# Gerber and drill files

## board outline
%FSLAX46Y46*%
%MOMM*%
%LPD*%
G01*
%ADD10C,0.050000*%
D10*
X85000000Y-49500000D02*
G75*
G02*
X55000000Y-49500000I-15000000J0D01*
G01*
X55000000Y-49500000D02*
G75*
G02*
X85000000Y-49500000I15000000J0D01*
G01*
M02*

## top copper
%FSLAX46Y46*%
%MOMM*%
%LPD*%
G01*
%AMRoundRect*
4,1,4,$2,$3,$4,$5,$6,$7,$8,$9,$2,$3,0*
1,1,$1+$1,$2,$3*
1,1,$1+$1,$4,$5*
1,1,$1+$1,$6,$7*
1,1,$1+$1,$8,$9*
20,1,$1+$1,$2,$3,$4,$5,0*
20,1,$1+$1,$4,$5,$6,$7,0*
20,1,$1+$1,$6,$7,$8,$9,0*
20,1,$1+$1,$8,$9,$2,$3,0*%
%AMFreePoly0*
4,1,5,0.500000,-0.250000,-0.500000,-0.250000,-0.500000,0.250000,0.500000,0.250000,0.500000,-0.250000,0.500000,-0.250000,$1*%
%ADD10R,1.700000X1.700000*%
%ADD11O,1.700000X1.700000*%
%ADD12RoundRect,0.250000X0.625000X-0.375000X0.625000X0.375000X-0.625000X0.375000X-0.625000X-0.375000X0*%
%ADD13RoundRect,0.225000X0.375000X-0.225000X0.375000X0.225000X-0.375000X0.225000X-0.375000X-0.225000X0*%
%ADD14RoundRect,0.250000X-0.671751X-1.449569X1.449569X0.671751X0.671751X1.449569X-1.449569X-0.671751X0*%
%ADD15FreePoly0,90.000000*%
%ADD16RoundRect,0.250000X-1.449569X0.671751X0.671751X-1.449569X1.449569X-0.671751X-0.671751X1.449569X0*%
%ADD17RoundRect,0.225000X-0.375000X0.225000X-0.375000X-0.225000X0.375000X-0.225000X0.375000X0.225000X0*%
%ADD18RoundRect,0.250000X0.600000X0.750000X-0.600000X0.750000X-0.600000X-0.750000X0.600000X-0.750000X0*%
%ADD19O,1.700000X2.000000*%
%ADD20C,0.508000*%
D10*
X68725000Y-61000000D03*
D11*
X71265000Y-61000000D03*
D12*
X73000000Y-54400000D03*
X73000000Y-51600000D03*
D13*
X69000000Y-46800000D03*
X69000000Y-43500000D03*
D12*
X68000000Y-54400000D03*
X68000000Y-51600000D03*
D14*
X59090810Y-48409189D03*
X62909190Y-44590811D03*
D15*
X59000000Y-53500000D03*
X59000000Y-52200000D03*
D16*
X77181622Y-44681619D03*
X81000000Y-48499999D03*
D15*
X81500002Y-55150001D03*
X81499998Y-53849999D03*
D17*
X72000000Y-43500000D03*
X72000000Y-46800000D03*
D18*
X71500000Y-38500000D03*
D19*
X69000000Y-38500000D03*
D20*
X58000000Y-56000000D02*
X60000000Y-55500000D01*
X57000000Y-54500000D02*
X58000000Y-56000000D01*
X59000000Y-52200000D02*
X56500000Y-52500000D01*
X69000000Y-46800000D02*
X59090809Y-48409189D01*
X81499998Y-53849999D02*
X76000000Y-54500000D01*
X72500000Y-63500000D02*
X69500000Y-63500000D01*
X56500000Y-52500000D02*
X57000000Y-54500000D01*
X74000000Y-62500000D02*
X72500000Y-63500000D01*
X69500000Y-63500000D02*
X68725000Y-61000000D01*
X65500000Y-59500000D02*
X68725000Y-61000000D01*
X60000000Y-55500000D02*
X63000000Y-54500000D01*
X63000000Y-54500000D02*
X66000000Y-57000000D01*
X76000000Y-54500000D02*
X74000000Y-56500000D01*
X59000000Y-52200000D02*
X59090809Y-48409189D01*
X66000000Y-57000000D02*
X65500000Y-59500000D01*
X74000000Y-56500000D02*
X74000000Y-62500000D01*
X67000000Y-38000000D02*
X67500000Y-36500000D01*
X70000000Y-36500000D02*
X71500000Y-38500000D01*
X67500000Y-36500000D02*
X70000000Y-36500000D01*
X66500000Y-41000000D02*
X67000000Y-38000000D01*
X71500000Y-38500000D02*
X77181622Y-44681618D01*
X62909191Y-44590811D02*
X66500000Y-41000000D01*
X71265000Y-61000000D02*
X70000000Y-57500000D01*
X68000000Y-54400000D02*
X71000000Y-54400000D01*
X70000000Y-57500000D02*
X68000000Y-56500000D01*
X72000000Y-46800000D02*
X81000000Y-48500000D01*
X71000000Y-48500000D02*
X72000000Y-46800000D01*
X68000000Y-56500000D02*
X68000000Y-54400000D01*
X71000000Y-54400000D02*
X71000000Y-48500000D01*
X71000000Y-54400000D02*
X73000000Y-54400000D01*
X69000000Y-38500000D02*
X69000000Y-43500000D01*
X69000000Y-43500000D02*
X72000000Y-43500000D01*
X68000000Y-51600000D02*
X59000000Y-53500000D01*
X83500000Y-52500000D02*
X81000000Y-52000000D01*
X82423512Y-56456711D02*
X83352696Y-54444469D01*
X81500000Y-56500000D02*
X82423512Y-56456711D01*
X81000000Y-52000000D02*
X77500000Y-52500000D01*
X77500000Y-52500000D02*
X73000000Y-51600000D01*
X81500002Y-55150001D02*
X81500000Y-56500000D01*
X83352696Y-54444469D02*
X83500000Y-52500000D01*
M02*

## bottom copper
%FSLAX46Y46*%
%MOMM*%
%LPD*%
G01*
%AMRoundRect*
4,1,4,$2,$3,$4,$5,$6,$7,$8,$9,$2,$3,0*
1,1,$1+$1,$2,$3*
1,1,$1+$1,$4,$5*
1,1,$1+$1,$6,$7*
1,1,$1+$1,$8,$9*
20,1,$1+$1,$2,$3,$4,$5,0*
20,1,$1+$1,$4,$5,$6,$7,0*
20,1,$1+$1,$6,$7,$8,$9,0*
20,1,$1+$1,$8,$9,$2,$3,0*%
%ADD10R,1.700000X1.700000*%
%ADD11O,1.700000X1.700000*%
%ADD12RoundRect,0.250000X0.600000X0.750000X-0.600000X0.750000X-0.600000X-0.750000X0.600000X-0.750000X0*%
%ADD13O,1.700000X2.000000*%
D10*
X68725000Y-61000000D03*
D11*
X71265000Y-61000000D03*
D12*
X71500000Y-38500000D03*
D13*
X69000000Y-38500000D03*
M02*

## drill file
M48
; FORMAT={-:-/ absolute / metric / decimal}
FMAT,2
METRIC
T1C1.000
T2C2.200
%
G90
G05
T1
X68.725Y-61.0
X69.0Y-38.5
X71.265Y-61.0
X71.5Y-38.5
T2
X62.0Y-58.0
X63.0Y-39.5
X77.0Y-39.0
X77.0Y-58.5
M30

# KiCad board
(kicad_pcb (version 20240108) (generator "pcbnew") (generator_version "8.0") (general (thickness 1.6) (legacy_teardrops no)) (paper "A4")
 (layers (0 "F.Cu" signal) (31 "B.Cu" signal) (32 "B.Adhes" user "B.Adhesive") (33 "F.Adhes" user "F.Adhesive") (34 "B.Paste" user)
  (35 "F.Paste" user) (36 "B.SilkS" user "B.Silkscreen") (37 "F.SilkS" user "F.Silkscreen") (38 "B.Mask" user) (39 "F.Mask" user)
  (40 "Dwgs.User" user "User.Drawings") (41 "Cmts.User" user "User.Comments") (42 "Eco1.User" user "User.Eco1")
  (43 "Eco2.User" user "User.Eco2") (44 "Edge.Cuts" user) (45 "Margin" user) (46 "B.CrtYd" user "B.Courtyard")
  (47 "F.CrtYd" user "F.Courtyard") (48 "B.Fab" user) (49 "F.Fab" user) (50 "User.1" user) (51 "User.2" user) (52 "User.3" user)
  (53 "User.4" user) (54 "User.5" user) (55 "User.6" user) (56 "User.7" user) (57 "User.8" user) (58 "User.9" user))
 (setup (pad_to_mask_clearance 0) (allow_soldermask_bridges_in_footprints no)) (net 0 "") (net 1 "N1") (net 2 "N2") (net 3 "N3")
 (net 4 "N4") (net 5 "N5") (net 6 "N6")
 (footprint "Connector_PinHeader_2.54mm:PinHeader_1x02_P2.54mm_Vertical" (layer "F.Cu") (at 68.725 61 90)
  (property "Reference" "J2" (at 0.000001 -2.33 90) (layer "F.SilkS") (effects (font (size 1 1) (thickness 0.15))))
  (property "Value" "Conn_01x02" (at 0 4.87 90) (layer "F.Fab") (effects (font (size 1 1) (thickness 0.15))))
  (pad "1" thru_hole rect (at 0 0 90) (size 1.7 1.7) (drill 1) (layers "*.Cu" "*.Mask") (remove_unused_layers no) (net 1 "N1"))
  (pad "2" thru_hole oval (at 0 2.54 90) (size 1.7 1.7) (drill 1) (layers "*.Cu" "*.Mask") (remove_unused_layers no) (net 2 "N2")))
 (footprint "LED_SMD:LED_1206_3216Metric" (layer "F.Cu") (at 73 53 90)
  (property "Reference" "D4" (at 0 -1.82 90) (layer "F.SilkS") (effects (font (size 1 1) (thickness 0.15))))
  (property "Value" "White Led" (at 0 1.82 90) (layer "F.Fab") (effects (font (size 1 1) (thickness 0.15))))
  (pad "1" smd roundrect (at -1.4 0 90) (size 1.25 1.75) (layers "F.Cu" "F.Paste" "F.Mask") (roundrect_rratio 0.2) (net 2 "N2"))
  (pad "2" smd roundrect (at 1.4 0 90) (size 1.25 1.75) (layers "F.Cu" "F.Paste" "F.Mask") (roundrect_rratio 0.2) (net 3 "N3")))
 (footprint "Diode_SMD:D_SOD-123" (layer "F.Cu") (at 69 45.15 90)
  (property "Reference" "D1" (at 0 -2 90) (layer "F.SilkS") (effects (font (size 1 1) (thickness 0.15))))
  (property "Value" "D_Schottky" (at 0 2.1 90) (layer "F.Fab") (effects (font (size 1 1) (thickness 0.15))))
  (pad "1" smd roundrect (at -1.65 0 90) (size 0.9 1.2) (layers "F.Cu" "F.Paste" "F.Mask") (roundrect_rratio 0.25) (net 1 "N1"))
  (pad "2" smd roundrect (at 1.65 0 90) (size 0.9 1.2) (layers "F.Cu" "F.Paste" "F.Mask") (roundrect_rratio 0.25) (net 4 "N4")))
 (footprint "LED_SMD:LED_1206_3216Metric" (layer "F.Cu") (at 68 53 90)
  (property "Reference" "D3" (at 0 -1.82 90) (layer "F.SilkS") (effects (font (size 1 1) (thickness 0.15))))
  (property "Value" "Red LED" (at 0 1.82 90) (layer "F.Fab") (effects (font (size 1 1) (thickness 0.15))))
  (pad "1" smd roundrect (at -1.4 0 90) (size 1.25 1.75) (layers "F.Cu" "F.Paste" "F.Mask") (roundrect_rratio 0.2) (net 2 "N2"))
  (pad "2" smd roundrect (at 1.4 0 90) (size 1.25 1.75) (layers "F.Cu" "F.Paste" "F.Mask") (roundrect_rratio 0.2) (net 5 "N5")))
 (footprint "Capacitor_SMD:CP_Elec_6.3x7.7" (layer "F.Cu") (at 61 46.5 45)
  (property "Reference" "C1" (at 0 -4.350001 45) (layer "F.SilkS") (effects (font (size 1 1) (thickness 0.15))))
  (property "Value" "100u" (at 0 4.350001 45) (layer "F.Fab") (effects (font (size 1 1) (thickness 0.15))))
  (pad "1" smd roundrect (at -2.700002 -0.000001 45) (size 3.5 1.6) (layers "F.Cu" "F.Paste" "F.Mask") (roundrect_rratio 0.15625)
   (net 1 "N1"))
  (pad "2" smd roundrect (at 2.700002 0.000001 45) (size 3.5 1.6) (layers "F.Cu" "F.Paste" "F.Mask") (roundrect_rratio 0.15625) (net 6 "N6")))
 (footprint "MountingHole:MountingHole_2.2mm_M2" (layer "F.Cu") (at 62 58)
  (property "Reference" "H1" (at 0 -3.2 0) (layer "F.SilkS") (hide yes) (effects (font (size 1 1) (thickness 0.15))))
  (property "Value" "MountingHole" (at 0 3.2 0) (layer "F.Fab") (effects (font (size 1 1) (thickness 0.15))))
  (pad "" np_thru_hole circle (at 0 0) (size 2.2 2.2) (drill 2.2) (layers "*.Cu" "*.Mask")))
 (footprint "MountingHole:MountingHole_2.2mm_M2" (layer "F.Cu") (at 77 39)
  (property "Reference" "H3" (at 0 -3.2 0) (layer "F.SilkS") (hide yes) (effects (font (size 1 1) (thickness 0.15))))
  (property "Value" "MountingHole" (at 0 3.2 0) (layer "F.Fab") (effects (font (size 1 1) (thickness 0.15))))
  (pad "" np_thru_hole circle (at 0 0) (size 2.2 2.2) (drill 2.2) (layers "*.Cu" "*.Mask")))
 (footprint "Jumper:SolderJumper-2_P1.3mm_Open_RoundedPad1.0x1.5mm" (layer "F.Cu") (at 59 52.85 90)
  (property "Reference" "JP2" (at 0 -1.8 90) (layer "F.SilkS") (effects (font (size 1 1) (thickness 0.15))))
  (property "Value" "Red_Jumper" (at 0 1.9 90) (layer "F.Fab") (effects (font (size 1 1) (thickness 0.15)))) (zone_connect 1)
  (pad "1" smd custom (at -0.65 0 90) (size 1 0.5) (layers "F.Cu" "F.Mask") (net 5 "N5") (zone_connect 2) (thermal_bridge_angle 45)
   (options (clearance outline) (anchor rect)) (primitives))
  (pad "2" smd custom (at 0.65 0 90) (size 1 0.5) (layers "F.Cu" "F.Mask") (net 1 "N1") (zone_connect 2) (thermal_bridge_angle 45)
   (options (clearance outline) (anchor rect)) (primitives)))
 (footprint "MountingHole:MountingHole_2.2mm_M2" (layer "F.Cu") (at 77 58.5)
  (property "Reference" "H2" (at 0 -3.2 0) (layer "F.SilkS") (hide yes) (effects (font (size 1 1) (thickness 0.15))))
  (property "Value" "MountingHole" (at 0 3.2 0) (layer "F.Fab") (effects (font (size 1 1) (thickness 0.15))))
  (pad "" np_thru_hole circle (at 0 0) (size 2.2 2.2) (drill 2.2) (layers "*.Cu" "*.Mask")))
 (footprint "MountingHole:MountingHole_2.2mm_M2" (layer "F.Cu") (at 63 39.5)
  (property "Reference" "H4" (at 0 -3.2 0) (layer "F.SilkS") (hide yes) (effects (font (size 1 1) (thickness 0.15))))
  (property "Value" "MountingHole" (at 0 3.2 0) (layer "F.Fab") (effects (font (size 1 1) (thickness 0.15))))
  (pad "" np_thru_hole circle (at 0 0) (size 2.2 2.2) (drill 2.2) (layers "*.Cu" "*.Mask")))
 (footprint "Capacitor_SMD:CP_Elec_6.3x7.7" (layer "F.Cu") (at 79.090811 46.590809 -45)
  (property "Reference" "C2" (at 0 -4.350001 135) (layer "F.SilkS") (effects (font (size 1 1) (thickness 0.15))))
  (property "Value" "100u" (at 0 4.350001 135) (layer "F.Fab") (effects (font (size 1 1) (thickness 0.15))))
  (pad "1" smd roundrect (at -2.700002 -0.000001 315) (size 3.5 1.6) (layers "F.Cu" "F.Paste" "F.Mask") (roundrect_rratio 0.15625)
   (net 6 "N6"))
  (pad "2" smd roundrect (at 2.700002 0.000001 315) (size 3.5 1.6) (layers "F.Cu" "F.Paste" "F.Mask") (roundrect_rratio 0.15625)
   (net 2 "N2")))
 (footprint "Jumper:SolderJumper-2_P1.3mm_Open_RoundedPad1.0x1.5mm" (layer "F.Cu") (at 81.5 54.5 90)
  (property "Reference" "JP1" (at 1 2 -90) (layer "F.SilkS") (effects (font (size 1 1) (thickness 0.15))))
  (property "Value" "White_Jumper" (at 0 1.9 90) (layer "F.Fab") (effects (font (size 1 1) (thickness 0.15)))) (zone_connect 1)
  (pad "1" smd custom (at -0.650001 0.000002 90) (size 1 0.5) (layers "F.Cu" "F.Mask") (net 3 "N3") (zone_connect 2)
   (thermal_bridge_angle 45) (options (clearance outline) (anchor rect)) (primitives))
  (pad "2" smd custom (at 0.650001 -0.000002 90) (size 1 0.5) (layers "F.Cu" "F.Mask") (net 1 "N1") (zone_connect 2)
   (thermal_bridge_angle 45) (options (clearance outline) (anchor rect)) (primitives)))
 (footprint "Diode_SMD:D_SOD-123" (layer "F.Cu") (at 72 45.15 -90)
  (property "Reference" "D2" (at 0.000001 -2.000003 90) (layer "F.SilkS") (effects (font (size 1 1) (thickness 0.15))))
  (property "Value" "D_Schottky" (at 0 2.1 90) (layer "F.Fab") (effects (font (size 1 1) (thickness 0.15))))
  (pad "1" smd roundrect (at -1.65 0 270) (size 0.9 1.2) (layers "F.Cu" "F.Paste" "F.Mask") (roundrect_rratio 0.25) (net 4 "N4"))
  (pad "2" smd roundrect (at 1.65 0 270) (size 0.9 1.2) (layers "F.Cu" "F.Paste" "F.Mask") (roundrect_rratio 0.25) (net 2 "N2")))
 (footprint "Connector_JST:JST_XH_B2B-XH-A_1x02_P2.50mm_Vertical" (layer "B.Cu") (at 71.5 38.5 180)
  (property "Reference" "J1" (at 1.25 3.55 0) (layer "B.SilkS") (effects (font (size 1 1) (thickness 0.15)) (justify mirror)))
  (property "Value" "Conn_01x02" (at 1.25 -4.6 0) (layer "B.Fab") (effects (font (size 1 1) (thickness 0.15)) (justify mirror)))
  (pad "1" thru_hole roundrect (at 0 0 180) (size 1.7 2) (drill 1) (layers "*.Cu" "*.Mask") (remove_unused_layers no)
   (roundrect_rratio 0.147059) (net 6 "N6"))
  (pad "2" thru_hole oval (at 2.5 0 180) (size 1.7 2) (drill 1) (layers "*.Cu" "*.Mask") (remove_unused_layers no) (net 4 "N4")))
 (gr_circle (center 70 49.5) (end 85 49.5) (stroke (width 0.05) (type default)) (fill none) (layer "Edge.Cuts"))
 (segment (start 58 56) (end 60 55.5) (width 0.508) (layer "F.Cu") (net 1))
 (segment (start 57 54.5) (end 58 56) (width 0.508) (layer "F.Cu") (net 1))
 (segment (start 59 52.2) (end 56.5 52.5) (width 0.508) (layer "F.Cu") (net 1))
 (segment (start 69 46.8) (end 59.090809 48.409189) (width 0.508) (layer "F.Cu") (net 1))
 (segment (start 81.499998 53.849999) (end 76 54.5) (width 0.508) (layer "F.Cu") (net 1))
 (segment (start 72.5 63.5) (end 69.5 63.5) (width 0.508) (layer "F.Cu") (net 1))
 (segment (start 56.5 52.5) (end 57 54.5) (width 0.508) (layer "F.Cu") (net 1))
 (segment (start 74 62.5) (end 72.5 63.5) (width 0.508) (layer "F.Cu") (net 1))
 (segment (start 69.5 63.5) (end 68.725 61) (width 0.508) (layer "F.Cu") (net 1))
 (segment (start 65.5 59.5) (end 68.725 61) (width 0.508) (layer "F.Cu") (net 1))
 (segment (start 60 55.5) (end 63 54.5) (width 0.508) (layer "F.Cu") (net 1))
 (segment (start 63 54.5) (end 66 57) (width 0.508) (layer "F.Cu") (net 1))
 (segment (start 76 54.5) (end 74 56.5) (width 0.508) (layer "F.Cu") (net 1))
 (segment (start 59 52.2) (end 59.090809 48.409189) (width 0.508) (layer "F.Cu") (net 1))
 (segment (start 66 57) (end 65.5 59.5) (width 0.508) (layer "F.Cu") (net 1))
 (segment (start 74 56.5) (end 74 62.5) (width 0.508) (layer "F.Cu") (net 1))
 (segment (start 67 38) (end 67.5 36.5) (width 0.508) (layer "F.Cu") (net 6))
 (segment (start 70 36.5) (end 71.5 38.5) (width 0.508) (layer "F.Cu") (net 6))
 (segment (start 67.5 36.5) (end 70 36.5) (width 0.508) (layer "F.Cu") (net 6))
 (segment (start 66.5 41) (end 67 38) (width 0.508) (layer "F.Cu") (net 6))
 (segment (start 71.5 38.5) (end 77.181622 44.681618) (width 0.508) (layer "F.Cu") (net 6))
 (segment (start 62.909191 44.590811) (end 66.5 41) (width 0.508) (layer "F.Cu") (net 6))
 (segment (start 71.265 61) (end 70 57.5) (width 0.508) (layer "F.Cu") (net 2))
 (segment (start 68 54.4) (end 71 54.4) (width 0.508) (layer "F.Cu") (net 2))
 (segment (start 70 57.5) (end 68 56.5) (width 0.508) (layer "F.Cu") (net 2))
 (segment (start 72 46.8) (end 81 48.5) (width 0.508) (layer "F.Cu") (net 2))
 (segment (start 71 48.5) (end 72 46.8) (width 0.508) (layer "F.Cu") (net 2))
 (segment (start 68 56.5) (end 68 54.4) (width 0.508) (layer "F.Cu") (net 2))
 (segment (start 71 54.4) (end 71 48.5) (width 0.508) (layer "F.Cu") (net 2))
 (segment (start 71 54.4) (end 73 54.4) (width 0.508) (layer "F.Cu") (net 2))
 (segment (start 69 38.5) (end 69 43.5) (width 0.508) (layer "F.Cu") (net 4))
 (segment (start 69 43.5) (end 72 43.5) (width 0.508) (layer "F.Cu") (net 4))
 (segment (start 68 51.6) (end 59 53.5) (width 0.508) (layer "F.Cu") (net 5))
 (segment (start 83.5 52.5) (end 81 52) (width 0.508) (layer "F.Cu") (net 3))
 (segment (start 82.423512 56.456711) (end 83.352696 54.444469) (width 0.508) (layer "F.Cu") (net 3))
 (segment (start 81.5 56.5) (end 82.423512 56.456711) (width 0.508) (layer "F.Cu") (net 3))
 (segment (start 81 52) (end 77.5 52.5) (width 0.508) (layer "F.Cu") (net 3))
 (segment (start 77.5 52.5) (end 73 51.6) (width 0.508) (layer "F.Cu") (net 3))
 (segment (start 81.500002 55.150001) (end 81.5 56.5) (width 0.508) (layer "F.Cu") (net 3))
 (segment (start 83.352696 54.444469) (end 83.5 52.5) (width 0.508) (layer "F.Cu") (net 3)))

